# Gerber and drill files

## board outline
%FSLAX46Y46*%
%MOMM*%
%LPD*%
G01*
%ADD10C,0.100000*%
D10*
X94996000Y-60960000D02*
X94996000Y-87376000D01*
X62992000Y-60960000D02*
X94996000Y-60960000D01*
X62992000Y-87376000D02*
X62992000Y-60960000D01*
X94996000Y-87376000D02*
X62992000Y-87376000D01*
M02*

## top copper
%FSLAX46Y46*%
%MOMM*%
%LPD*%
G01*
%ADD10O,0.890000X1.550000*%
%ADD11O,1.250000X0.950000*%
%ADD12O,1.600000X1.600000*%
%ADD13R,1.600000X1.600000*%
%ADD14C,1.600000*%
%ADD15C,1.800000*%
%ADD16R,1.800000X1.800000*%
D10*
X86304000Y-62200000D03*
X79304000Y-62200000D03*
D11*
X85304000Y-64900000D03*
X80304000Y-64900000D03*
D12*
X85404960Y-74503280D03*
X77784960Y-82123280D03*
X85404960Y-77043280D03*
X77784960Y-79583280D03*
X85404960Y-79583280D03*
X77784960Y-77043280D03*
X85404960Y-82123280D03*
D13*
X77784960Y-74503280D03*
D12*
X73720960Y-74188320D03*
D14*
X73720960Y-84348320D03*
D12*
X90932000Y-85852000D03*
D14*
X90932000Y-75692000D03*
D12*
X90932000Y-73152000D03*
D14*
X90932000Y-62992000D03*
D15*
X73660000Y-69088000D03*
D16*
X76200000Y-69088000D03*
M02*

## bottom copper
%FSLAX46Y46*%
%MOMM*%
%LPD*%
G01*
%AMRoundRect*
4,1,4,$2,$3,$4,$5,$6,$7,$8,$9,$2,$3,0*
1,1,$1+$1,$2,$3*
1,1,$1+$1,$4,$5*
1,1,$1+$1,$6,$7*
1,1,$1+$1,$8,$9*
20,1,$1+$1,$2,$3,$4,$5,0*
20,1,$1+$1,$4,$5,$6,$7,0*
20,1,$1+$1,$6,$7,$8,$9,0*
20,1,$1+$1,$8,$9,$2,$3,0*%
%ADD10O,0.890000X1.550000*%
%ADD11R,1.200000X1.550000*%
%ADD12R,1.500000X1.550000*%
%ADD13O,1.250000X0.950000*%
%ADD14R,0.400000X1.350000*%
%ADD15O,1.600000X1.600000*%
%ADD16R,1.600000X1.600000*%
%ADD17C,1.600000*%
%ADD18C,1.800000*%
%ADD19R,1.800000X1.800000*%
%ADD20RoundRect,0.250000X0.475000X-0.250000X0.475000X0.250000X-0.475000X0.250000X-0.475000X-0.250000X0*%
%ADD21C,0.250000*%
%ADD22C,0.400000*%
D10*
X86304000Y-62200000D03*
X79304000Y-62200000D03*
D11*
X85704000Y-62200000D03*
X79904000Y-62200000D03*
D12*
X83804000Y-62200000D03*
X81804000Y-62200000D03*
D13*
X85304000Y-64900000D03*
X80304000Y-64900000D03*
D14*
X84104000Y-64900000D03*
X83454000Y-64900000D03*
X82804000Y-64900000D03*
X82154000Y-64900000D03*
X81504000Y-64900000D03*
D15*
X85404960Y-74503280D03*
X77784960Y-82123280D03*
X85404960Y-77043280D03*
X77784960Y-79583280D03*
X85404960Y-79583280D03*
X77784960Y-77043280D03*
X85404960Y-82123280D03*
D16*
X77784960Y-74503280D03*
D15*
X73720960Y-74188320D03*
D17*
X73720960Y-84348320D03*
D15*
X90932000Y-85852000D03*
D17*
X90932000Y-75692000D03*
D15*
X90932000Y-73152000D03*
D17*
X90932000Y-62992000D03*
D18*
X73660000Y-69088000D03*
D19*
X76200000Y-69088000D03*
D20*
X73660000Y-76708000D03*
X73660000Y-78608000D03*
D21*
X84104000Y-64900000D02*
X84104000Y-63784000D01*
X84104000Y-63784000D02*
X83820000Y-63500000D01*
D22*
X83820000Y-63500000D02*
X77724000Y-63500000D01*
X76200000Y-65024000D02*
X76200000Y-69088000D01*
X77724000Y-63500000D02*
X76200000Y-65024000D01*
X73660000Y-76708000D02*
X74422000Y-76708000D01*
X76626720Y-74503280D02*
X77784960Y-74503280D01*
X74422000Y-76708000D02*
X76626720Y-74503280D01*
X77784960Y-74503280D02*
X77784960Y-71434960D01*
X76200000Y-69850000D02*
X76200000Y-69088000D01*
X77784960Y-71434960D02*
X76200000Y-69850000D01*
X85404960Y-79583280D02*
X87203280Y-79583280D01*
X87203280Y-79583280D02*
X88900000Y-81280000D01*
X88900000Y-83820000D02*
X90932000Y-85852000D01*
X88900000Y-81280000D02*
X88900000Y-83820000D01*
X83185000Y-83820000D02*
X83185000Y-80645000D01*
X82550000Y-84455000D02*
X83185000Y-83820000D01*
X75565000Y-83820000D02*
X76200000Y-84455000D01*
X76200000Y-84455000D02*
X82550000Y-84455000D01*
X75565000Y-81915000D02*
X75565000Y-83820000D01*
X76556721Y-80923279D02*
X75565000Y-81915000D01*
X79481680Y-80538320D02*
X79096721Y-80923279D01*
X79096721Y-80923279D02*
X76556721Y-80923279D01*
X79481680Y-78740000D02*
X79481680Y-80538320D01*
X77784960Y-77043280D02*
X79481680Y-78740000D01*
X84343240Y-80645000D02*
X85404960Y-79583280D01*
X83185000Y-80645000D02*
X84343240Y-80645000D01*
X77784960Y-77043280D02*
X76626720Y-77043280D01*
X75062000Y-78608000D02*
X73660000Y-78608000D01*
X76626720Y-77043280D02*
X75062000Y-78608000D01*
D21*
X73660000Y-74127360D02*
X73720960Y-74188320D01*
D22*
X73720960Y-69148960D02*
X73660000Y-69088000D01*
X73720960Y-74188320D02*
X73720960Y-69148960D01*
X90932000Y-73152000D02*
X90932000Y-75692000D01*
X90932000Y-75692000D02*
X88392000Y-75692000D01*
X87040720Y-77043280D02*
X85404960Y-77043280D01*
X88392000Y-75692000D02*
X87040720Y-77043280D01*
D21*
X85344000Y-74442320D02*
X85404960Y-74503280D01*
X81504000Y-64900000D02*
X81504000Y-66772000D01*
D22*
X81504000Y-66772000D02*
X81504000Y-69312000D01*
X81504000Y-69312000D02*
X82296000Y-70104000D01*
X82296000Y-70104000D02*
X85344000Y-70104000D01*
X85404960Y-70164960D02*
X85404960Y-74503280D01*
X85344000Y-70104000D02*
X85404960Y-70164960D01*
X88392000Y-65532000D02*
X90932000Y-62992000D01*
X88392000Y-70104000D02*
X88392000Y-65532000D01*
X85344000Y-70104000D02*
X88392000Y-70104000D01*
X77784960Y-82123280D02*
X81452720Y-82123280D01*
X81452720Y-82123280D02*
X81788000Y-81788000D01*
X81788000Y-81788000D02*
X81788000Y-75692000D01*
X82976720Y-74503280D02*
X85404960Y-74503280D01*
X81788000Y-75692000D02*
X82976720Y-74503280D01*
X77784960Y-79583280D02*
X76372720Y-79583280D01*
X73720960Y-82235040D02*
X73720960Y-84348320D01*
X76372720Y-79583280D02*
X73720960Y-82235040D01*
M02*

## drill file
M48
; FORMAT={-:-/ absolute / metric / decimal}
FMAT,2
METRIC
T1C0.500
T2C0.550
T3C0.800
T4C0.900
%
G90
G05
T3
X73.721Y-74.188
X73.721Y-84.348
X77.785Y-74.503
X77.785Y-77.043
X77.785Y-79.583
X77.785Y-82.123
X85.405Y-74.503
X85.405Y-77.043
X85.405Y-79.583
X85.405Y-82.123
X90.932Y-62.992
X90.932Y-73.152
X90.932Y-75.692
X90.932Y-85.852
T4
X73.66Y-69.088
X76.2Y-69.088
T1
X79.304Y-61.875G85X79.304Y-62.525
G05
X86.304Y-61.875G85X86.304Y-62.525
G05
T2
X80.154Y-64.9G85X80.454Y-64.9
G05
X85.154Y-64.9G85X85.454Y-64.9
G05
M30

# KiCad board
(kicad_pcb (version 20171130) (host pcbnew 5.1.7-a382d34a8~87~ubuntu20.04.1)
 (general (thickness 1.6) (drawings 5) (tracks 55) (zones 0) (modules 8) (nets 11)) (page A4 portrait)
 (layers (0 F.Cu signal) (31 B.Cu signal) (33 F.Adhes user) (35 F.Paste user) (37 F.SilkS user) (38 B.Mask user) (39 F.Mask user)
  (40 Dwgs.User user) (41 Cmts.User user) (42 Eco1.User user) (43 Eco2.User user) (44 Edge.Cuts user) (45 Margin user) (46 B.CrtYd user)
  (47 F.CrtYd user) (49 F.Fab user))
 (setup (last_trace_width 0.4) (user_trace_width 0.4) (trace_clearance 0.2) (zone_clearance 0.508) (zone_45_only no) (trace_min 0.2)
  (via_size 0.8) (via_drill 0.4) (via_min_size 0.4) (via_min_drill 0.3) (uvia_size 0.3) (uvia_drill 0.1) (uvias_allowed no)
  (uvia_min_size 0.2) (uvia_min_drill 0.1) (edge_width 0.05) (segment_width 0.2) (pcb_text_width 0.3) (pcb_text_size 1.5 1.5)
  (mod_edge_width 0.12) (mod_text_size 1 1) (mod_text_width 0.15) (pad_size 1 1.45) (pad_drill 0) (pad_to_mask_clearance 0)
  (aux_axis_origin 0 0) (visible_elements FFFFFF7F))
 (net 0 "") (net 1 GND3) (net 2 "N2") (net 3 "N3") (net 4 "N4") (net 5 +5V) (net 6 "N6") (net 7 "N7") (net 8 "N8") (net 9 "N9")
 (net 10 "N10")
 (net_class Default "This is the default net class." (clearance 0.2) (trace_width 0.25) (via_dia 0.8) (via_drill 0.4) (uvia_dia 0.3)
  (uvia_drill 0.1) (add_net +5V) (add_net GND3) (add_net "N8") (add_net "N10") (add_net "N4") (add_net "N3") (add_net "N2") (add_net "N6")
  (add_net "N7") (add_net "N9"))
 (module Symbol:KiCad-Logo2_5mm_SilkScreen (layer F.Cu) (at 66.548 77.216 90)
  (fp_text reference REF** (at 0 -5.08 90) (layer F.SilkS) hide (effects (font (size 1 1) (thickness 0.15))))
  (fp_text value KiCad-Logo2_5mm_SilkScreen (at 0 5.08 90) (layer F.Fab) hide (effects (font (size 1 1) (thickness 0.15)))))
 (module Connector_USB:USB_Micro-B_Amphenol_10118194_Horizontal (layer B.Cu) (at 82.804 63.5)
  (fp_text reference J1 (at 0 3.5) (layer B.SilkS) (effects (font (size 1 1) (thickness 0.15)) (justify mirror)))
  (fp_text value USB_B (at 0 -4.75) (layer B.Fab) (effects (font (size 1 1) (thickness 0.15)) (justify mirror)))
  (pad "" smd oval (at 2.5 1.4) (size 1.25 0.95) (layers B.Paste))
  (pad "" smd oval (at -2.5 1.4) (size 1.25 0.95) (layers B.Paste))
  (pad 6 thru_hole oval (at 3.5 -1.3) (size 0.89 1.55) (drill oval 0.5 1.15) (layers *.Cu *.Mask))
  (pad 6 thru_hole oval (at -3.5 -1.3) (size 0.89 1.55) (drill oval 0.5 1.15) (layers *.Cu *.Mask))
  (pad 6 smd rect (at 2.9 -1.3) (size 1.2 1.55) (layers B.Cu B.Paste B.Mask))
  (pad 6 smd rect (at -2.9 -1.3) (size 1.2 1.55) (layers B.Cu B.Paste B.Mask))
  (pad "" smd oval (at 3.5 -1.3) (size 0.89 1.55) (layers B.Paste))
  (pad 6 smd rect (at 1 -1.3) (size 1.5 1.55) (layers B.Cu B.Paste B.Mask))
  (pad 6 smd rect (at -1 -1.3) (size 1.5 1.55) (layers B.Cu B.Paste B.Mask))
  (pad 6 thru_hole oval (at 2.5 1.4) (size 1.25 0.95) (drill oval 0.85 0.55) (layers *.Cu *.Mask))
  (pad "" smd oval (at -3.5 -1.3) (size 0.89 1.55) (layers B.Paste))
  (pad 6 thru_hole oval (at -2.5 1.4) (size 1.25 0.95) (drill oval 0.85 0.55) (layers *.Cu *.Mask))
  (pad 5 smd rect (at 1.3 1.4) (size 0.4 1.35) (layers B.Cu B.Paste B.Mask) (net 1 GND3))
  (pad 4 smd rect (at 0.65 1.4) (size 0.4 1.35) (layers B.Cu B.Paste B.Mask) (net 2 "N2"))
  (pad 3 smd rect (at 0 1.4) (size 0.4 1.35) (layers B.Cu B.Paste B.Mask) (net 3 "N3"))
  (pad 2 smd rect (at -0.65 1.4) (size 0.4 1.35) (layers B.Cu B.Paste B.Mask) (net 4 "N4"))
  (pad 1 smd rect (at -1.3 1.4) (size 0.4 1.35) (layers B.Cu B.Paste B.Mask) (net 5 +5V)))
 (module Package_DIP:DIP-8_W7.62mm (layer F.Cu) (at 77.78496 74.50328)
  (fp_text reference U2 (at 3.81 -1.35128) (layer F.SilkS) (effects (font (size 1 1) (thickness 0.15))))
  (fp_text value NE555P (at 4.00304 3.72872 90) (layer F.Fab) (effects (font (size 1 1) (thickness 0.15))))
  (pad 8 thru_hole oval (at 7.62 0) (size 1.6 1.6) (drill 0.8) (layers *.Cu *.Mask) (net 5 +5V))
  (pad 4 thru_hole oval (at 0 7.62) (size 1.6 1.6) (drill 0.8) (layers *.Cu *.Mask) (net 5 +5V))
  (pad 7 thru_hole oval (at 7.62 2.54) (size 1.6 1.6) (drill 0.8) (layers *.Cu *.Mask) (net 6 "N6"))
  (pad 3 thru_hole oval (at 0 5.08) (size 1.6 1.6) (drill 0.8) (layers *.Cu *.Mask) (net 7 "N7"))
  (pad 6 thru_hole oval (at 7.62 5.08) (size 1.6 1.6) (drill 0.8) (layers *.Cu *.Mask) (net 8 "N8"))
  (pad 2 thru_hole oval (at 0 2.54) (size 1.6 1.6) (drill 0.8) (layers *.Cu *.Mask) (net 8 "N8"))
  (pad 5 thru_hole oval (at 7.62 7.62) (size 1.6 1.6) (drill 0.8) (layers *.Cu *.Mask) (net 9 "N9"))
  (pad 1 thru_hole rect (at 0 0) (size 1.6 1.6) (drill 0.8) (layers *.Cu *.Mask) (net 1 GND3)))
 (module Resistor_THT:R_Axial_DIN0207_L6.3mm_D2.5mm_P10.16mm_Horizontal (layer F.Cu) (at 73.72096 84.34832 90)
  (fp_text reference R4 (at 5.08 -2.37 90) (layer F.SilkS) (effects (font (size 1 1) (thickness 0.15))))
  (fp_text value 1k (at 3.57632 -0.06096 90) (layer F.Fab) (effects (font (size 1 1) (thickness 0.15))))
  (pad 2 thru_hole oval (at 10.16 0 90) (size 1.6 1.6) (drill 0.8) (layers *.Cu *.Mask) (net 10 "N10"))
  (pad 1 thru_hole circle (at 0 0 90) (size 1.6 1.6) (drill 0.8) (layers *.Cu *.Mask) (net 7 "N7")))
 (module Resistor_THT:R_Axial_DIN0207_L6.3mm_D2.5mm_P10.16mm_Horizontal (layer F.Cu) (at 90.932 75.692 270)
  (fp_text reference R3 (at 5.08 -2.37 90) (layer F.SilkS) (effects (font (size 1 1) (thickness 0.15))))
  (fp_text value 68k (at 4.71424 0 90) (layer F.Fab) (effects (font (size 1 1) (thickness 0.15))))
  (pad 2 thru_hole oval (at 10.16 0 270) (size 1.6 1.6) (drill 0.8) (layers *.Cu *.Mask) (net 8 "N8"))
  (pad 1 thru_hole circle (at 0 0 270) (size 1.6 1.6) (drill 0.8) (layers *.Cu *.Mask) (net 6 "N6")))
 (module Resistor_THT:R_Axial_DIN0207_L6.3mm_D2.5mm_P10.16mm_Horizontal (layer F.Cu) (at 90.932 62.992 270)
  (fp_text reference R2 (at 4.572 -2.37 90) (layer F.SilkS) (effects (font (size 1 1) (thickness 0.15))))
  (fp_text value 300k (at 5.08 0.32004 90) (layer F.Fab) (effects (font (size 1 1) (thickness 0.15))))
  (pad 2 thru_hole oval (at 10.16 0 270) (size 1.6 1.6) (drill 0.8) (layers *.Cu *.Mask) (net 6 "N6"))
  (pad 1 thru_hole circle (at 0 0 270) (size 1.6 1.6) (drill 0.8) (layers *.Cu *.Mask) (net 5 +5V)))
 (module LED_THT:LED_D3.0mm (layer F.Cu) (at 76.2 69.088 180)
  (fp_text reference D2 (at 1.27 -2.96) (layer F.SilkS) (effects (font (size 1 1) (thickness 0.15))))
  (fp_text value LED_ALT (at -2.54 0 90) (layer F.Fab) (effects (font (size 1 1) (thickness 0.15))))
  (pad 2 thru_hole circle (at 2.54 0 180) (size 1.8 1.8) (drill 0.9) (layers *.Cu *.Mask) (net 10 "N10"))
  (pad 1 thru_hole rect (at 0 0 180) (size 1.8 1.8) (drill 0.9) (layers *.Cu *.Mask) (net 1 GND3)))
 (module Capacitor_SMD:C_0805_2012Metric (layer B.Cu) (at 73.66 77.658 90)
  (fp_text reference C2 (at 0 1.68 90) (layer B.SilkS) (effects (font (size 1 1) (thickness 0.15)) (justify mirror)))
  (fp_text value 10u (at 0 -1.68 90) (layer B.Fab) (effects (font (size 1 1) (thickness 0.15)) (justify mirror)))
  (pad 2 smd roundrect (at 0.95 0 90) (size 1 1.45) (layers B.Cu B.Paste B.Mask) (roundrect_rratio 0.25) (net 1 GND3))
  (pad 1 smd roundrect (at -0.95 0 90) (size 1 1.45) (layers B.Cu B.Paste B.Mask) (roundrect_rratio 0.25) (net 8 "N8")))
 (gr_line (start 94.996 60.96) (end 94.996 87.376) (layer Edge.Cuts) (width 0.1))
 (gr_line (start 62.992 60.96) (end 94.996 60.96) (layer Edge.Cuts) (width 0.1))
 (gr_line (start 62.992 87.376) (end 62.992 60.96) (layer Edge.Cuts) (width 0.1))
 (gr_line (start 94.996 87.376) (end 62.992 87.376) (layer Edge.Cuts) (width 0.1))
 (segment (start 84.104 64.9) (end 84.104 63.784) (width 0.25) (layer B.Cu) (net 1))
 (segment (start 84.104 63.784) (end 83.82 63.5) (width 0.25) (layer B.Cu) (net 1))
 (segment (start 83.82 63.5) (end 77.724 63.5) (width 0.4) (layer B.Cu) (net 1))
 (segment (start 76.2 65.024) (end 76.2 69.088) (width 0.4) (layer B.Cu) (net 1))
 (segment (start 77.724 63.5) (end 76.2 65.024) (width 0.4) (layer B.Cu) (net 1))
 (segment (start 73.66 76.708) (end 74.422 76.708) (width 0.4) (layer B.Cu) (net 1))
 (segment (start 76.62672 74.50328) (end 77.78496 74.50328) (width 0.4) (layer B.Cu) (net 1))
 (segment (start 74.422 76.708) (end 76.62672 74.50328) (width 0.4) (layer B.Cu) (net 1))
 (segment (start 77.78496 74.50328) (end 77.78496 71.43496) (width 0.4) (layer B.Cu) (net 1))
 (segment (start 76.2 69.85) (end 76.2 69.088) (width 0.4) (layer B.Cu) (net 1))
 (segment (start 77.78496 71.43496) (end 76.2 69.85) (width 0.4) (layer B.Cu) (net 1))
 (segment (start 85.40496 79.58328) (end 87.20328 79.58328) (width 0.4) (layer B.Cu) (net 8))
 (segment (start 87.20328 79.58328) (end 88.9 81.28) (width 0.4) (layer B.Cu) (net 8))
 (segment (start 88.9 83.82) (end 90.932 85.852) (width 0.4) (layer B.Cu) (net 8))
 (segment (start 88.9 81.28) (end 88.9 83.82) (width 0.4) (layer B.Cu) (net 8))
 (segment (start 83.185 83.82) (end 83.185 80.645) (width 0.4) (layer B.Cu) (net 8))
 (segment (start 82.55 84.455) (end 83.185 83.82) (width 0.4) (layer B.Cu) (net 8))
 (segment (start 75.565 83.82) (end 76.2 84.455) (width 0.4) (layer B.Cu) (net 8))
 (segment (start 76.2 84.455) (end 82.55 84.455) (width 0.4) (layer B.Cu) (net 8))
 (segment (start 75.565 81.915) (end 75.565 83.82) (width 0.4) (layer B.Cu) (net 8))
 (segment (start 76.556721 80.923279) (end 75.565 81.915) (width 0.4) (layer B.Cu) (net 8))
 (segment (start 79.48168 80.53832) (end 79.096721 80.923279) (width 0.4) (layer B.Cu) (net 8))
 (segment (start 79.096721 80.923279) (end 76.556721 80.923279) (width 0.4) (layer B.Cu) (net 8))
 (segment (start 79.48168 78.74) (end 79.48168 80.53832) (width 0.4) (layer B.Cu) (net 8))
 (segment (start 77.78496 77.04328) (end 79.48168 78.74) (width 0.4) (layer B.Cu) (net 8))
 (segment (start 84.34324 80.645) (end 85.40496 79.58328) (width 0.4) (layer B.Cu) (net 8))
 (segment (start 83.185 80.645) (end 84.34324 80.645) (width 0.4) (layer B.Cu) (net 8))
 (segment (start 77.78496 77.04328) (end 76.62672 77.04328) (width 0.4) (layer B.Cu) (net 8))
 (segment (start 75.062 78.608) (end 73.66 78.608) (width 0.4) (layer B.Cu) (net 8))
 (segment (start 76.62672 77.04328) (end 75.062 78.608) (width 0.4) (layer B.Cu) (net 8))
 (segment (start 73.66 74.12736) (end 73.72096 74.18832) (width 0.25) (layer B.Cu) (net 10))
 (segment (start 73.72096 69.14896) (end 73.66 69.088) (width 0.4) (layer B.Cu) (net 10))
 (segment (start 73.72096 74.18832) (end 73.72096 69.14896) (width 0.4) (layer B.Cu) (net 10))
 (segment (start 90.932 73.152) (end 90.932 75.692) (width 0.4) (layer B.Cu) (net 6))
 (segment (start 90.932 75.692) (end 88.392 75.692) (width 0.4) (layer B.Cu) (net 6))
 (segment (start 87.04072 77.04328) (end 85.40496 77.04328) (width 0.4) (layer B.Cu) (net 6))
 (segment (start 88.392 75.692) (end 87.04072 77.04328) (width 0.4) (layer B.Cu) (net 6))
 (segment (start 85.344 74.44232) (end 85.40496 74.50328) (width 0.25) (layer B.Cu) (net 5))
 (segment (start 81.504 64.9) (end 81.504 66.772) (width 0.25) (layer B.Cu) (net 5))
 (segment (start 81.504 66.772) (end 81.504 69.312) (width 0.4) (layer B.Cu) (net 5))
 (segment (start 81.504 69.312) (end 82.296 70.104) (width 0.4) (layer B.Cu) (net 5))
 (segment (start 82.296 70.104) (end 85.344 70.104) (width 0.4) (layer B.Cu) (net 5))
 (segment (start 85.40496 70.16496) (end 85.40496 74.50328) (width 0.4) (layer B.Cu) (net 5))
 (segment (start 85.344 70.104) (end 85.40496 70.16496) (width 0.4) (layer B.Cu) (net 5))
 (segment (start 88.392 65.532) (end 90.932 62.992) (width 0.4) (layer B.Cu) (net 5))
 (segment (start 88.392 70.104) (end 88.392 65.532) (width 0.4) (layer B.Cu) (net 5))
 (segment (start 85.344 70.104) (end 88.392 70.104) (width 0.4) (layer B.Cu) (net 5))
 (segment (start 77.78496 82.12328) (end 81.45272 82.12328) (width 0.4) (layer B.Cu) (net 5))
 (segment (start 81.45272 82.12328) (end 81.788 81.788) (width 0.4) (layer B.Cu) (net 5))
 (segment (start 81.788 81.788) (end 81.788 75.692) (width 0.4) (layer B.Cu) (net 5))
 (segment (start 82.97672 74.50328) (end 85.40496 74.50328) (width 0.4) (layer B.Cu) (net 5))
 (segment (start 81.788 75.692) (end 82.97672 74.50328) (width 0.4) (layer B.Cu) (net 5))
 (segment (start 77.78496 79.58328) (end 76.37272 79.58328) (width 0.4) (layer B.Cu) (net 7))
 (segment (start 73.72096 82.23504) (end 73.72096 84.34832) (width 0.4) (layer B.Cu) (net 7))
 (segment (start 76.37272 79.58328) (end 73.72096 82.23504) (width 0.4) (layer B.Cu) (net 7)))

